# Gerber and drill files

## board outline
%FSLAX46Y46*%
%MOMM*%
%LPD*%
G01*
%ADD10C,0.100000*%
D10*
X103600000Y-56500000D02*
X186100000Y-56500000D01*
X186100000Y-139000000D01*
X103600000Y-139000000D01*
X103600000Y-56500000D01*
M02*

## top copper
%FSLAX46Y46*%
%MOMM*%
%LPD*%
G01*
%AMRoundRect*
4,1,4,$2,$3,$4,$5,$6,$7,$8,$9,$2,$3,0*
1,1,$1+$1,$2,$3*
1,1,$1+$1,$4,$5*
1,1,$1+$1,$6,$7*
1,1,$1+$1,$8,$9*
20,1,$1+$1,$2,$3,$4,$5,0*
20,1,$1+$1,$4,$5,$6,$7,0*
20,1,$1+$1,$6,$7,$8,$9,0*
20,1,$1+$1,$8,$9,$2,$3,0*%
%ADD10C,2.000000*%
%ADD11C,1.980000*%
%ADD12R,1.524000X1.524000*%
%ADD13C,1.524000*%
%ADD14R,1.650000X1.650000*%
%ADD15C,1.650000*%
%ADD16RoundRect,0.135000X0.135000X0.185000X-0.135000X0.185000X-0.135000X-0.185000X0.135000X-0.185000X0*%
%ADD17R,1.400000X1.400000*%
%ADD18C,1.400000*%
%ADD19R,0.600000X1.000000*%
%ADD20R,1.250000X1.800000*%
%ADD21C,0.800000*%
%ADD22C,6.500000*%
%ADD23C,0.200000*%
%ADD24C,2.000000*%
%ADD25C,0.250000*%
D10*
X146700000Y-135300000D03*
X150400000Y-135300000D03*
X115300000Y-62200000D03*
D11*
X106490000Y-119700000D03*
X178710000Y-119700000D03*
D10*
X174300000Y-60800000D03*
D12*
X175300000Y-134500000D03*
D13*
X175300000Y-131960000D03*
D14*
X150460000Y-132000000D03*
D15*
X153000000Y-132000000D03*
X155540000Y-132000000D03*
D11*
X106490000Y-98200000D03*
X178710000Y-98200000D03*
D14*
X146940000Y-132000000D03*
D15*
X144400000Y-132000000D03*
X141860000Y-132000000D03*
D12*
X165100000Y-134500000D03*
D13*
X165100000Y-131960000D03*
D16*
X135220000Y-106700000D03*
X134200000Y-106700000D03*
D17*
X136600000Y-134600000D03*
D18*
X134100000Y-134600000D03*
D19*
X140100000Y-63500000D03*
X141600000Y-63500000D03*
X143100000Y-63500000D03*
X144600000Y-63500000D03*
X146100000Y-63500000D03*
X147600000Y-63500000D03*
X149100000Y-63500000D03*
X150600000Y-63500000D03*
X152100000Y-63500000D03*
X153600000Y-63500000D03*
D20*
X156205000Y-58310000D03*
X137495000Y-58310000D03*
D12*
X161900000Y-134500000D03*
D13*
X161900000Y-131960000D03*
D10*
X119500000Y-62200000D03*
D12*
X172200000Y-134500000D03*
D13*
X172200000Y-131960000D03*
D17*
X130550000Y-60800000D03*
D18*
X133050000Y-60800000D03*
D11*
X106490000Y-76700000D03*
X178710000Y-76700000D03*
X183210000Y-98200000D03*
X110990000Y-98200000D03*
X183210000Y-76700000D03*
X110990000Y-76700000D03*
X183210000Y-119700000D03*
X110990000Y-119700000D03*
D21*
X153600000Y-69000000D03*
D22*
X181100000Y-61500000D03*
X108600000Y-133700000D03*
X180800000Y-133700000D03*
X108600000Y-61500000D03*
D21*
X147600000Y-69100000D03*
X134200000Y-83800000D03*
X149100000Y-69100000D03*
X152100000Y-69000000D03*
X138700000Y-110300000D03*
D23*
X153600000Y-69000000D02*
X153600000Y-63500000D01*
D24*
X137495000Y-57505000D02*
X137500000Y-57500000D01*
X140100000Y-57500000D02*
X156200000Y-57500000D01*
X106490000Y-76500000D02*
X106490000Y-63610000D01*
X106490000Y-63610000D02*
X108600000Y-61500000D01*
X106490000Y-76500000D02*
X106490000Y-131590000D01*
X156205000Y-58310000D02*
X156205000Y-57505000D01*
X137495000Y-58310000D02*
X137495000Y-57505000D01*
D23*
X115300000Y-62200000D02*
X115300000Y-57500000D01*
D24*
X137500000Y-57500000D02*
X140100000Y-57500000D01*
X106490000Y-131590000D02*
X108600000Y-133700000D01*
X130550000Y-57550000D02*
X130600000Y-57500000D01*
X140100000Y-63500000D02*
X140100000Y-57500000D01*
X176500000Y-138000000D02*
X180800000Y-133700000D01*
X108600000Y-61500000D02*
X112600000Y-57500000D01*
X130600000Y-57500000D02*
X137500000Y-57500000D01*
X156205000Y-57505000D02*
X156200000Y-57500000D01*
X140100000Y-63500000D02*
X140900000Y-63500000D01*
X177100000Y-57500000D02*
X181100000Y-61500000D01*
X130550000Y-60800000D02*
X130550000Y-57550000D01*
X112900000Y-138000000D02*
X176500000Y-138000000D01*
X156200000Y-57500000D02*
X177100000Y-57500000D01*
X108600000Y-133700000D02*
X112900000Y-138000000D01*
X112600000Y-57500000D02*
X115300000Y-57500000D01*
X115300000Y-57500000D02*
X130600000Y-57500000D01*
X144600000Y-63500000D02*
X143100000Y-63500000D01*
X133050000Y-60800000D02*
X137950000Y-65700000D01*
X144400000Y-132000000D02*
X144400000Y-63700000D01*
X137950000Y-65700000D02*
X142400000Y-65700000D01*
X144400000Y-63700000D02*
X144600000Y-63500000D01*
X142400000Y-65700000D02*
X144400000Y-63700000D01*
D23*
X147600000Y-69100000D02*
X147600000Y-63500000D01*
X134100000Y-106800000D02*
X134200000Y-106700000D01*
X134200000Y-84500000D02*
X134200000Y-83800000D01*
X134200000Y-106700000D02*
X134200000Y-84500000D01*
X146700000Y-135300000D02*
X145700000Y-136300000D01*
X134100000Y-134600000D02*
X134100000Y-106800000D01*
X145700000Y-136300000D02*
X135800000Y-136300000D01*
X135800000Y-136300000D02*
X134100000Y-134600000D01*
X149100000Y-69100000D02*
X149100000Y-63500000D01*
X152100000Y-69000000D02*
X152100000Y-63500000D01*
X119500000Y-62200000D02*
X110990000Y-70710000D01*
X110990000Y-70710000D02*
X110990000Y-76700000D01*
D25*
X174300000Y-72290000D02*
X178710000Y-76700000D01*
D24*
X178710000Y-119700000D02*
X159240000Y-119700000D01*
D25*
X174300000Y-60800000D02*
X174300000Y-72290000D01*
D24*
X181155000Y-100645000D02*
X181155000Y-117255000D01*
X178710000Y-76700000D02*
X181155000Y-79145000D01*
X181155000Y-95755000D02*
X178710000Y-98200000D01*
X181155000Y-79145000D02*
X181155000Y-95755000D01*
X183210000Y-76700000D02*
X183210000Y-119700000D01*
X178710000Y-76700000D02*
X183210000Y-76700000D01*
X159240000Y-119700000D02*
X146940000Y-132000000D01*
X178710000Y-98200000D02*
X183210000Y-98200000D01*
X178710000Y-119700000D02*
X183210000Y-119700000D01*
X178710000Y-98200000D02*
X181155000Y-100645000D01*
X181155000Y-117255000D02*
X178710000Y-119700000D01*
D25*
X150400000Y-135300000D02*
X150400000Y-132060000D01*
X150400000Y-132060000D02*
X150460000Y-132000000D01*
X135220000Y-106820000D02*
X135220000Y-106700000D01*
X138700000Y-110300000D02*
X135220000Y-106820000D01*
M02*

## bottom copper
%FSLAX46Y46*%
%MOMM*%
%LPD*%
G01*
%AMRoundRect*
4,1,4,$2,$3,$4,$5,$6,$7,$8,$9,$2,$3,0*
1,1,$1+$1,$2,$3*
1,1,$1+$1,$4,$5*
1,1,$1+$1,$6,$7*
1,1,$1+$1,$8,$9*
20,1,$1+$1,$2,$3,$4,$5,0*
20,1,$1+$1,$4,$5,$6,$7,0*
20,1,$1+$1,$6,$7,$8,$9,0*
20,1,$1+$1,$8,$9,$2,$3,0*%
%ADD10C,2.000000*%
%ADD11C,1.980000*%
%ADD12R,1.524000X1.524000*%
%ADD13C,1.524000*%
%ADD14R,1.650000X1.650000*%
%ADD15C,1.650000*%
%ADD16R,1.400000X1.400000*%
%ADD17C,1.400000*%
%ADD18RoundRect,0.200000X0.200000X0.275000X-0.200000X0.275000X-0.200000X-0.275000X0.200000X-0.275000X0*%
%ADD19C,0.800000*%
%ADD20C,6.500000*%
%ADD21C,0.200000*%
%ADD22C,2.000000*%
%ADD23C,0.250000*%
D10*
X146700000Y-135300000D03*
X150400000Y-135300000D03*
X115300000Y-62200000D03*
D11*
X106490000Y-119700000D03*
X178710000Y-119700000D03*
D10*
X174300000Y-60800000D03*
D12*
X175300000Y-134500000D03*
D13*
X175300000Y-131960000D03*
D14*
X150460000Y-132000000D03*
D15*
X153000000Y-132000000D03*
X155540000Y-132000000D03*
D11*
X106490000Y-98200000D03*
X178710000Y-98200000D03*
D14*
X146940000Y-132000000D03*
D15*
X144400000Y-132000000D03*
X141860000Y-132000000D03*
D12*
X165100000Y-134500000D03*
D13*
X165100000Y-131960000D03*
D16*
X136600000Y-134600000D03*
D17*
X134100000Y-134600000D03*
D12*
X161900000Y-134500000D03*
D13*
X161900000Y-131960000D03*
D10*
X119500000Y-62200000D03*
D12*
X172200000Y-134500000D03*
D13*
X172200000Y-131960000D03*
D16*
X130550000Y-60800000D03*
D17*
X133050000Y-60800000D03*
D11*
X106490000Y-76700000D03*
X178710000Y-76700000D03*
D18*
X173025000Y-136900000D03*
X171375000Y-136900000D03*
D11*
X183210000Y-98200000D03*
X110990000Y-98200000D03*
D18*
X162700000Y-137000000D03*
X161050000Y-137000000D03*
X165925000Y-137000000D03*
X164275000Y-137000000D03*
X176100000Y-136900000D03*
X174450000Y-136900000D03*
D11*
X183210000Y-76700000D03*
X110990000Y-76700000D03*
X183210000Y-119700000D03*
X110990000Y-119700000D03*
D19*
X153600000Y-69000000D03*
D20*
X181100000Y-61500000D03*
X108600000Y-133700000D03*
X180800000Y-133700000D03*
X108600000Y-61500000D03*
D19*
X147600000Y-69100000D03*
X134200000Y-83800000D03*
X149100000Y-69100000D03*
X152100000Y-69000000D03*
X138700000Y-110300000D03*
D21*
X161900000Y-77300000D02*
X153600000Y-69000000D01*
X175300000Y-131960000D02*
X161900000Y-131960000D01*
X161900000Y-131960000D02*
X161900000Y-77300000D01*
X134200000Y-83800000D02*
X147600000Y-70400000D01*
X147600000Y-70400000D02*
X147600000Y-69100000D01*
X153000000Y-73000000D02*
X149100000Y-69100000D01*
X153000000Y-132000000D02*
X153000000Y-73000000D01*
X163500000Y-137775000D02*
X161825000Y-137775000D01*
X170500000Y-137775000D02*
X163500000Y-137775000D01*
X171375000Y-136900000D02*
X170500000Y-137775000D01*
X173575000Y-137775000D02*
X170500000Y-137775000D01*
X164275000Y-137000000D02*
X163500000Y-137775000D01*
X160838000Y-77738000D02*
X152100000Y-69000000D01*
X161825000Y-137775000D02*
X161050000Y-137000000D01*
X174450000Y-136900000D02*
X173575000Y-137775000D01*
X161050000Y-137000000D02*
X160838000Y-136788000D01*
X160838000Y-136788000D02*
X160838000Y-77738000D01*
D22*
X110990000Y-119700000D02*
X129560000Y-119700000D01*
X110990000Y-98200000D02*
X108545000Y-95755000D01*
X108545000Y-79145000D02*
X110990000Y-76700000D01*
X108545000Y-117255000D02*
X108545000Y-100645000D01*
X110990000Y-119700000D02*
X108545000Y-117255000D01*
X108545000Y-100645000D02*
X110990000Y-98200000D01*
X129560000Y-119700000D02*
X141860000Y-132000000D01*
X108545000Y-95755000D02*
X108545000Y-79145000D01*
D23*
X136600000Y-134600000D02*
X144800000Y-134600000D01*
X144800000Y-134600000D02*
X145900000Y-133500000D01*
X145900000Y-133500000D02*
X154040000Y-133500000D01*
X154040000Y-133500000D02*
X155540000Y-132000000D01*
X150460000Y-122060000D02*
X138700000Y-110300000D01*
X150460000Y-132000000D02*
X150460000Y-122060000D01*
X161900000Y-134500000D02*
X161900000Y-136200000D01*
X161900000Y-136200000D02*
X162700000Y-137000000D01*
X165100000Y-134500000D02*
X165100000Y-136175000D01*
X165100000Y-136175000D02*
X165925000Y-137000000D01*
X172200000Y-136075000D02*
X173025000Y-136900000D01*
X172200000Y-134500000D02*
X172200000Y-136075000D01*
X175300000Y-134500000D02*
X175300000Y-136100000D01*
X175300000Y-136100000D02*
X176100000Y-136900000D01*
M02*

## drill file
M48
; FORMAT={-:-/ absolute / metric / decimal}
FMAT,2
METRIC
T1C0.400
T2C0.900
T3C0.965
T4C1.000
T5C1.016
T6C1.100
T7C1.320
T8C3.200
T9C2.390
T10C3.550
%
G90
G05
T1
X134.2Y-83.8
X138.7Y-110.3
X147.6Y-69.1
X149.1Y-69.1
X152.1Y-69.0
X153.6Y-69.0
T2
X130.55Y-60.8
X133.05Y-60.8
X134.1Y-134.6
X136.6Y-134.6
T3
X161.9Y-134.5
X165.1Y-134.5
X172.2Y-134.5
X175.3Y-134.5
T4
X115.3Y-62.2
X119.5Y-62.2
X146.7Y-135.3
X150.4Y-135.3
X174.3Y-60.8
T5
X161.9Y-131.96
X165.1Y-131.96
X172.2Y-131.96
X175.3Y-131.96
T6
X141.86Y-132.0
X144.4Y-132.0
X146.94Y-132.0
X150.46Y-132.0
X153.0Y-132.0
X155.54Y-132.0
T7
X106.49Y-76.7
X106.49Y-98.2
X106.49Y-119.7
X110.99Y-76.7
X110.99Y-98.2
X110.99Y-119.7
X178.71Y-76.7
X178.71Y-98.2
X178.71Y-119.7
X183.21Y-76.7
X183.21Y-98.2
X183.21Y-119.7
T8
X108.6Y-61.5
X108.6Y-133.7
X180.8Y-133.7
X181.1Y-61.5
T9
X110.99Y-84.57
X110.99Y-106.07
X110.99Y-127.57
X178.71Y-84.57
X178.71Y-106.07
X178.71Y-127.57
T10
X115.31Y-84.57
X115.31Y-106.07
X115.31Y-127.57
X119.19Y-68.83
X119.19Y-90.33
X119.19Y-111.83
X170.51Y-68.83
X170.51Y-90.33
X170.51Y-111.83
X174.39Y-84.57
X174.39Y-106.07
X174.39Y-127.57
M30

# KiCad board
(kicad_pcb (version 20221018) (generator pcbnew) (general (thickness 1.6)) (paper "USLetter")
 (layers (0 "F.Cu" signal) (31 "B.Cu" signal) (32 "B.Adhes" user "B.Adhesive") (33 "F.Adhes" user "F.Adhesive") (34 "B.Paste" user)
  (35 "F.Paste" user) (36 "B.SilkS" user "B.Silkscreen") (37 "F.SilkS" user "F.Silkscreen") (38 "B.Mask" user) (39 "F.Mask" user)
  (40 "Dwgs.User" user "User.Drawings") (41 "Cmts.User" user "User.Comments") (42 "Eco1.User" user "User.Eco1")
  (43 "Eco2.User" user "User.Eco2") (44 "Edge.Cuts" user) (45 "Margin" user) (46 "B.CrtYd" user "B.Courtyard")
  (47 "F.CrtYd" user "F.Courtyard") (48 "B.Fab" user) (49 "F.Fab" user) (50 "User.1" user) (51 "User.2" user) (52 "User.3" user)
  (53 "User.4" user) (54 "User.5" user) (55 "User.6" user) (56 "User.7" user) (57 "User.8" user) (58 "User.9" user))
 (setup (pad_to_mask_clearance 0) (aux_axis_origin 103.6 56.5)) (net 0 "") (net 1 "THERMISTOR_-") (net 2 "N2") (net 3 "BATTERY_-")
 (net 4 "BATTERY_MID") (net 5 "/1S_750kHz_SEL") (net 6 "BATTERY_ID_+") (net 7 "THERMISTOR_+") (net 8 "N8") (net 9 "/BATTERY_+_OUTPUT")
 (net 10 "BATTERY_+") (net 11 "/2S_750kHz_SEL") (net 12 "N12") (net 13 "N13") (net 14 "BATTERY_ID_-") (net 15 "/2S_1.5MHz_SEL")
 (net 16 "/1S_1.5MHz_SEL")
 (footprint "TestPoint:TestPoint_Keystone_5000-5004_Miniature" (layer "F.Cu") (at 146.7 135.3)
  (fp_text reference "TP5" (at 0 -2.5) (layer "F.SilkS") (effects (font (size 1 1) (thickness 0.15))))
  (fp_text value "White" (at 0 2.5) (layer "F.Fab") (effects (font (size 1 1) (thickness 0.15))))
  (pad "1" thru_hole circle (at 0 0) (size 2 2) (drill 1) (layers "*.Cu" "*.Mask") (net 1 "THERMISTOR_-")))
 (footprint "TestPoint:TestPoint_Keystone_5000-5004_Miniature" (layer "F.Cu") (at 150.4 135.3)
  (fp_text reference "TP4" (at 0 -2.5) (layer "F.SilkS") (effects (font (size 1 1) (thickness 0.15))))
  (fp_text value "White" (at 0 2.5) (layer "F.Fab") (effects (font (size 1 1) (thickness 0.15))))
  (pad "1" thru_hole circle (at 0 0) (size 2 2) (drill 1) (layers "*.Cu" "*.Mask") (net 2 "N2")))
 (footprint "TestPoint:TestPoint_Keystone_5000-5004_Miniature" (layer "F.Cu") (at 115.3 62.2)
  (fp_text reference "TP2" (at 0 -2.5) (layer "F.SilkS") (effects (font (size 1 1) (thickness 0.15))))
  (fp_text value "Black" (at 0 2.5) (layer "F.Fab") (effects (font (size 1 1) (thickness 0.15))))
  (pad "1" thru_hole circle (at 0 0) (size 2 2) (drill 1) (layers "*.Cu" "*.Mask") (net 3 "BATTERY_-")))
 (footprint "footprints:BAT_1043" (layer "F.Cu") (at 142.6 119.7)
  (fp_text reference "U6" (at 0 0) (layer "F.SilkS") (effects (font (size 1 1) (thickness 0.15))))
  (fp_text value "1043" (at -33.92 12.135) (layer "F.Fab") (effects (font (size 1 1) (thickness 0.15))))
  (pad "" np_thru_hole circle (at -27.29 7.87) (size 3.55 3.55) (drill 3.55) (layers "*.Cu" "*.Mask"))
  (pad "" np_thru_hole circle (at 27.91 -7.87) (size 3.55 3.55) (drill 3.55) (layers "*.Cu" "*.Mask"))
  (pad "" np_thru_hole circle (at 36.11 7.87) (size 2.39 2.39) (drill 2.39) (layers "*.Cu" "*.Mask"))
  (pad "N" thru_hole circle (at -36.11 0) (size 1.98 1.98) (drill 1.32) (layers "*.Cu" "*.Mask") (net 3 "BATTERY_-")
   (solder_mask_margin 0.102))
  (pad "P" thru_hole circle (at 36.11 0) (size 1.98 1.98) (drill 1.32) (layers "*.Cu" "*.Mask") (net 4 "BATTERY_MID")
   (solder_mask_margin 0.102)))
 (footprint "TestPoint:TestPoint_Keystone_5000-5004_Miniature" (layer "F.Cu") (at 174.3 60.8)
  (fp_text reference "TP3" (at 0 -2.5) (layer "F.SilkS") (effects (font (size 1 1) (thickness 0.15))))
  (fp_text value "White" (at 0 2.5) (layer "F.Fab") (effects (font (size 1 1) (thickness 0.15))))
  (pad "1" thru_hole circle (at 0 0) (size 2 2) (drill 1) (layers "*.Cu" "*.Mask") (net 4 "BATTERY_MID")))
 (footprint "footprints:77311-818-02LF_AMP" (layer "F.Cu") (at 175.3 134.5 -90)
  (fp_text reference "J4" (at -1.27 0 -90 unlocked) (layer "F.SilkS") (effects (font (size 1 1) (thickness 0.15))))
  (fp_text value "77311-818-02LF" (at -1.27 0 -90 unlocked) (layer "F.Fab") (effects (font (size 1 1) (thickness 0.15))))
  (pad "1" thru_hole rect (at 0 0 270) (size 1.524 1.524) (drill 0.9652) (layers "*.Cu" "*.Mask") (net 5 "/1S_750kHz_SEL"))
  (pad "2" thru_hole circle (at -2.54 0 270) (size 1.524 1.524) (drill 1.016) (layers "*.Cu" "*.Mask") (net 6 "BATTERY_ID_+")))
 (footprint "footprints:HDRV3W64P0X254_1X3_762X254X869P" (layer "F.Cu") (at 150.46 132)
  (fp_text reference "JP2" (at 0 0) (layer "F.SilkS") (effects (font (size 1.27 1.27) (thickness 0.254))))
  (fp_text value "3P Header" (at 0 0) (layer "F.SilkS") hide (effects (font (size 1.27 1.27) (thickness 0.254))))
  (pad "1" thru_hole rect (at 0 0) (size 1.65 1.65) (drill 1.1) (layers "*.Cu" "*.Mask") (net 2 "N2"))
  (pad "2" thru_hole circle (at 2.54 0) (size 1.65 1.65) (drill 1.1) (layers "*.Cu" "*.Mask") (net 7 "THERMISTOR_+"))
  (pad "3" thru_hole circle (at 5.08 0) (size 1.65 1.65) (drill 1.1) (layers "*.Cu" "*.Mask") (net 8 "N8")))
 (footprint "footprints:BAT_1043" (layer "F.Cu") (at 142.6 98.2)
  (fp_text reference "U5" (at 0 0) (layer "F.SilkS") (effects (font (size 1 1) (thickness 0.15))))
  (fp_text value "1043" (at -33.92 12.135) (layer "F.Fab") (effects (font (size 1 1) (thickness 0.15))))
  (pad "" np_thru_hole circle (at -27.29 7.87) (size 3.55 3.55) (drill 3.55) (layers "*.Cu" "*.Mask"))
  (pad "" np_thru_hole circle (at 27.91 -7.87) (size 3.55 3.55) (drill 3.55) (layers "*.Cu" "*.Mask"))
  (pad "" np_thru_hole circle (at 36.11 7.87) (size 2.39 2.39) (drill 2.39) (layers "*.Cu" "*.Mask"))
  (pad "N" thru_hole circle (at -36.11 0) (size 1.98 1.98) (drill 1.32) (layers "*.Cu" "*.Mask") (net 3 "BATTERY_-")
   (solder_mask_margin 0.102))
  (pad "P" thru_hole circle (at 36.11 0) (size 1.98 1.98) (drill 1.32) (layers "*.Cu" "*.Mask") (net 4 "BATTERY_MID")
   (solder_mask_margin 0.102)))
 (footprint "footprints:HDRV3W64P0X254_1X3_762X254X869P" (layer "F.Cu") (at 146.94 132 180)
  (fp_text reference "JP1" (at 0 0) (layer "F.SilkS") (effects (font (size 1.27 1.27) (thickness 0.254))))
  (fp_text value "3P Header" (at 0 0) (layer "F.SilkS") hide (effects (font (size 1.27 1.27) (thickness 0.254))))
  (pad "1" thru_hole rect (at 0 0 180) (size 1.65 1.65) (drill 1.1) (layers "*.Cu" "*.Mask") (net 4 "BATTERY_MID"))
  (pad "2" thru_hole circle (at 2.54 0 180) (size 1.65 1.65) (drill 1.1) (layers "*.Cu" "*.Mask") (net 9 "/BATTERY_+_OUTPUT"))
  (pad "3" thru_hole circle (at 5.08 0 180) (size 1.65 1.65) (drill 1.1) (layers "*.Cu" "*.Mask") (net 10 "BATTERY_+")))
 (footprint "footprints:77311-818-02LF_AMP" (layer "F.Cu") (at 165.1 134.5 -90)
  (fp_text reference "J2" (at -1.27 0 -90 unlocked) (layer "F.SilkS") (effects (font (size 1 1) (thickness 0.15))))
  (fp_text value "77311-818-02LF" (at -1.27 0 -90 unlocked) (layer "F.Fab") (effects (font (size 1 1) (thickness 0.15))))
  (pad "1" thru_hole rect (at 0 0 270) (size 1.524 1.524) (drill 0.9652) (layers "*.Cu" "*.Mask") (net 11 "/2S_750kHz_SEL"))
  (pad "2" thru_hole circle (at -2.54 0 270) (size 1.524 1.524) (drill 1.016) (layers "*.Cu" "*.Mask") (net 6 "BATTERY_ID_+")))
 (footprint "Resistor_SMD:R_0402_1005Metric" (layer "F.Cu") (at 134.71 106.7 180)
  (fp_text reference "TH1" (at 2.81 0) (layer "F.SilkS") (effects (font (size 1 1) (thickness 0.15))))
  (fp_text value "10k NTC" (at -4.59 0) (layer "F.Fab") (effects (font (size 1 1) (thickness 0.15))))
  (pad "1" smd roundrect (at -0.51 0 180) (size 0.54 0.64) (layers "F.Cu" "F.Paste" "F.Mask") (roundrect_rratio 0.25) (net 2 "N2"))
  (pad "2" smd roundrect (at 0.51 0 180) (size 0.54 0.64) (layers "F.Cu" "F.Paste" "F.Mask") (roundrect_rratio 0.25) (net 1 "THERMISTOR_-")))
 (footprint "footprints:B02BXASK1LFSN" (layer "F.Cu") (at 136.6 134.6)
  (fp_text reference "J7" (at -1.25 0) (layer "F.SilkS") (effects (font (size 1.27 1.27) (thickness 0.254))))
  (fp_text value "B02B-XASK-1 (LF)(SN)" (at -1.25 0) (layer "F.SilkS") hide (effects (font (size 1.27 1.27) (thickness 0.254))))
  (pad "1" thru_hole rect (at 0 0) (size 1.4 1.4) (drill 0.9) (layers "*.Cu" "*.Mask") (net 8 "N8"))
  (pad "2" thru_hole circle (at -2.5 0) (size 1.4 1.4) (drill 0.9) (layers "*.Cu" "*.Mask") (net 1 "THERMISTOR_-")))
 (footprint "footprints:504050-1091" (layer "F.Cu") (at 153.6 63.5)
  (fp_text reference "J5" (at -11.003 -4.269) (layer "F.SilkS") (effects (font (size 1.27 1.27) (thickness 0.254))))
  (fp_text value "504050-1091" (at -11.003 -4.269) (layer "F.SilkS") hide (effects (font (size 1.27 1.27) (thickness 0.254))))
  (pad "1" smd rect (at -13.5 0) (size 0.6 1) (layers "F.Cu" "F.Paste" "F.Mask") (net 3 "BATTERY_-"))
  (pad "2" smd rect (at -12 0) (size 0.6 1) (layers "F.Cu" "F.Paste" "F.Mask") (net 3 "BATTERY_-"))
  (pad "3" smd rect (at -10.5 0) (size 0.6 1) (layers "F.Cu" "F.Paste" "F.Mask") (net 9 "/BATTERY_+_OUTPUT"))
  (pad "4" smd rect (at -9 0) (size 0.6 1) (layers "F.Cu" "F.Paste" "F.Mask") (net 9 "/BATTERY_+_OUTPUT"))
  (pad "5" smd rect (at -7.5 0) (size 0.6 1) (layers "F.Cu" "F.Paste" "F.Mask") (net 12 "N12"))
  (pad "6" smd rect (at -6 0) (size 0.6 1) (layers "F.Cu" "F.Paste" "F.Mask") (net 1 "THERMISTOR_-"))
  (pad "7" smd rect (at -4.5 0) (size 0.6 1) (layers "F.Cu" "F.Paste" "F.Mask") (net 7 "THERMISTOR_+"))
  (pad "8" smd rect (at -3 0) (size 0.6 1) (layers "F.Cu" "F.Paste" "F.Mask") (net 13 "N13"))
  (pad "9" smd rect (at -1.5 0) (size 0.6 1) (layers "F.Cu" "F.Paste" "F.Mask") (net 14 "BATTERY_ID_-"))
  (pad "10" smd rect (at 0 0) (size 0.6 1) (layers "F.Cu" "F.Paste" "F.Mask") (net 6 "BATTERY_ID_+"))
  (pad "11" smd rect (at 2.605 -5.19) (size 1.25 1.8) (layers "F.Cu" "F.Paste" "F.Mask") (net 3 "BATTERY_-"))
  (pad "12" smd rect (at -16.105 -5.19) (size 1.25 1.8) (layers "F.Cu" "F.Paste" "F.Mask") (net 3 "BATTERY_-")))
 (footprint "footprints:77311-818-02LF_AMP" (layer "F.Cu") (at 161.9 134.5 -90)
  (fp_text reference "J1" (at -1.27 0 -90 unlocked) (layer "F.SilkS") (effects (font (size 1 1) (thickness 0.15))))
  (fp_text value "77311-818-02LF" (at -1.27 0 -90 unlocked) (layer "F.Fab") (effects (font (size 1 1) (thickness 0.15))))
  (pad "1" thru_hole rect (at 0 0 270) (size 1.524 1.524) (drill 0.9652) (layers "*.Cu" "*.Mask") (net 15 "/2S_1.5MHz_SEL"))
  (pad "2" thru_hole circle (at -2.54 0 270) (size 1.524 1.524) (drill 1.016) (layers "*.Cu" "*.Mask") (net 6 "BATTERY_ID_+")))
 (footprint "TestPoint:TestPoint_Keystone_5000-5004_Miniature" (layer "F.Cu") (at 119.5 62.2)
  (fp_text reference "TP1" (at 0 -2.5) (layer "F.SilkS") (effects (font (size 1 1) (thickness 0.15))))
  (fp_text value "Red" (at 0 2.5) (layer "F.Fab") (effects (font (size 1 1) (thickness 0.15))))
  (pad "1" thru_hole circle (at 0 0) (size 2 2) (drill 1) (layers "*.Cu" "*.Mask") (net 10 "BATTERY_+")))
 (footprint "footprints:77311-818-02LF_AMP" (layer "F.Cu") (at 172.2 134.5 -90)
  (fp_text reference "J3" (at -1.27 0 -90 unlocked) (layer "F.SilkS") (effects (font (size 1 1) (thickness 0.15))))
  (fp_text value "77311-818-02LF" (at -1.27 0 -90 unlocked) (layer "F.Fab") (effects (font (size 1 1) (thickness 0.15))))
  (pad "1" thru_hole rect (at 0 0 270) (size 1.524 1.524) (drill 0.9652) (layers "*.Cu" "*.Mask") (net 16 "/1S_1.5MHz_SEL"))
  (pad "2" thru_hole circle (at -2.54 0 270) (size 1.524 1.524) (drill 1.016) (layers "*.Cu" "*.Mask") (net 6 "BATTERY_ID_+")))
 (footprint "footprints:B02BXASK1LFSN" (layer "F.Cu") (at 130.55 60.8 180)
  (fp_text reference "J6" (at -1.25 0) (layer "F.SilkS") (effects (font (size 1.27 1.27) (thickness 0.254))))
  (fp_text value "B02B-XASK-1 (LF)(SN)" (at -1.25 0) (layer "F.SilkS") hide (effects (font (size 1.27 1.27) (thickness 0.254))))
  (pad "1" thru_hole rect (at 0 0 180) (size 1.4 1.4) (drill 0.9) (layers "*.Cu" "*.Mask") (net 3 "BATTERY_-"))
  (pad "2" thru_hole circle (at -2.5 0 180) (size 1.4 1.4) (drill 0.9) (layers "*.Cu" "*.Mask") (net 9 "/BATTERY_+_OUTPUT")))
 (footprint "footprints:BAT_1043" (layer "F.Cu") (at 142.6 76.7)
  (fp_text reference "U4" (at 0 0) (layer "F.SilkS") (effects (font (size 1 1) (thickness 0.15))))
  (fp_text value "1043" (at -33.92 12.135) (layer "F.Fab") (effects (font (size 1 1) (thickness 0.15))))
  (pad "" np_thru_hole circle (at -27.29 7.87) (size 3.55 3.55) (drill 3.55) (layers "*.Cu" "*.Mask"))
  (pad "" np_thru_hole circle (at 27.91 -7.87) (size 3.55 3.55) (drill 3.55) (layers "*.Cu" "*.Mask"))
  (pad "" np_thru_hole circle (at 36.11 7.87) (size 2.39 2.39) (drill 2.39) (layers "*.Cu" "*.Mask"))
  (pad "N" thru_hole circle (at -36.11 0) (size 1.98 1.98) (drill 1.32) (layers "*.Cu" "*.Mask") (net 3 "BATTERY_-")
   (solder_mask_margin 0.102))
  (pad "P" thru_hole circle (at 36.11 0) (size 1.98 1.98) (drill 1.32) (layers "*.Cu" "*.Mask") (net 4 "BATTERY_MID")
   (solder_mask_margin 0.102)))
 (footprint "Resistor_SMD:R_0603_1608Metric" (layer "B.Cu") (at 172.2 136.9 180)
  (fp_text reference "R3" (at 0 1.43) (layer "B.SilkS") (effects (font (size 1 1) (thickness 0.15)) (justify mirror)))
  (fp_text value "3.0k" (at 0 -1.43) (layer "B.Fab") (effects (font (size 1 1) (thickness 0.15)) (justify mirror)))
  (pad "1" smd roundrect (at -0.825 0 180) (size 0.8 0.95) (layers "B.Cu" "B.Paste" "B.Mask") (roundrect_rratio 0.25)
   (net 16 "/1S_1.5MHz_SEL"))
  (pad "2" smd roundrect (at 0.825 0 180) (size 0.8 0.95) (layers "B.Cu" "B.Paste" "B.Mask") (roundrect_rratio 0.25) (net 14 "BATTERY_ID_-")))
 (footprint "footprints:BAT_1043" (layer "B.Cu") (at 147.1 98.2 180)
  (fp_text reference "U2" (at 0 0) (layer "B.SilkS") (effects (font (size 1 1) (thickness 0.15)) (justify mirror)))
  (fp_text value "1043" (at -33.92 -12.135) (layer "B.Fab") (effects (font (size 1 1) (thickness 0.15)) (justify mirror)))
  (pad "" np_thru_hole circle (at -27.29 -7.87 180) (size 3.55 3.55) (drill 3.55) (layers "*.Cu" "*.Mask"))
  (pad "" np_thru_hole circle (at 27.91 7.87 180) (size 3.55 3.55) (drill 3.55) (layers "*.Cu" "*.Mask"))
  (pad "" np_thru_hole circle (at 36.11 -7.87 180) (size 2.39 2.39) (drill 2.39) (layers "*.Cu" "*.Mask"))
  (pad "N" thru_hole circle (at -36.11 0 180) (size 1.98 1.98) (drill 1.32) (layers "*.Cu" "*.Mask") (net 4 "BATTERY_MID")
   (solder_mask_margin 0.102))
  (pad "P" thru_hole circle (at 36.11 0 180) (size 1.98 1.98) (drill 1.32) (layers "*.Cu" "*.Mask") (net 10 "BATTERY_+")
   (solder_mask_margin 0.102)))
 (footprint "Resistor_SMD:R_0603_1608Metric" (layer "B.Cu") (at 161.875 137 180)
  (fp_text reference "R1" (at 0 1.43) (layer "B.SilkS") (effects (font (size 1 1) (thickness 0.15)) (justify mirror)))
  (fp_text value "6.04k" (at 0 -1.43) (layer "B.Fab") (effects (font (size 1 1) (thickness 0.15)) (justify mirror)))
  (pad "1" smd roundrect (at -0.825 0 180) (size 0.8 0.95) (layers "B.Cu" "B.Paste" "B.Mask") (roundrect_rratio 0.25)
   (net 15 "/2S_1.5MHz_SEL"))
  (pad "2" smd roundrect (at 0.825 0 180) (size 0.8 0.95) (layers "B.Cu" "B.Paste" "B.Mask") (roundrect_rratio 0.25) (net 14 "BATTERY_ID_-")))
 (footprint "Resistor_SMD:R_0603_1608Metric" (layer "B.Cu") (at 165.1 137 180)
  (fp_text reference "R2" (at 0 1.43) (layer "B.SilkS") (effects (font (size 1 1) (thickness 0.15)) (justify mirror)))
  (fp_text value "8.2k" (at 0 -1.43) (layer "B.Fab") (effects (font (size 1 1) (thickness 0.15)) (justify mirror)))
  (pad "1" smd roundrect (at -0.825 0 180) (size 0.8 0.95) (layers "B.Cu" "B.Paste" "B.Mask") (roundrect_rratio 0.25)
   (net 11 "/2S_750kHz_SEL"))
  (pad "2" smd roundrect (at 0.825 0 180) (size 0.8 0.95) (layers "B.Cu" "B.Paste" "B.Mask") (roundrect_rratio 0.25) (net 14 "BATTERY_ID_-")))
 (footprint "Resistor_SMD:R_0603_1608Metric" (layer "B.Cu") (at 175.275 136.9 180)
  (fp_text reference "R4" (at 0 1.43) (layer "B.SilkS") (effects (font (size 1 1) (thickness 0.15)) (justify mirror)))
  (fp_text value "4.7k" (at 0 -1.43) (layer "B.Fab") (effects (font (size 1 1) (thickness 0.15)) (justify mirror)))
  (pad "1" smd roundrect (at -0.825 0 180) (size 0.8 0.95) (layers "B.Cu" "B.Paste" "B.Mask") (roundrect_rratio 0.25)
   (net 5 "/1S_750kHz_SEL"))
  (pad "2" smd roundrect (at 0.825 0 180) (size 0.8 0.95) (layers "B.Cu" "B.Paste" "B.Mask") (roundrect_rratio 0.25) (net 14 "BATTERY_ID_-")))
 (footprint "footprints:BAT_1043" (layer "B.Cu") (at 147.1 76.7 180)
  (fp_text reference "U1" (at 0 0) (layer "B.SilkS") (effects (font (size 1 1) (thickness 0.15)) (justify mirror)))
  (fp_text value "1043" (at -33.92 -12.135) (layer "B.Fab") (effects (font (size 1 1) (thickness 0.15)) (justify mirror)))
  (pad "" np_thru_hole circle (at -27.29 -7.87 180) (size 3.55 3.55) (drill 3.55) (layers "*.Cu" "*.Mask"))
  (pad "" np_thru_hole circle (at 27.91 7.87 180) (size 3.55 3.55) (drill 3.55) (layers "*.Cu" "*.Mask"))
  (pad "" np_thru_hole circle (at 36.11 -7.87 180) (size 2.39 2.39) (drill 2.39) (layers "*.Cu" "*.Mask"))
  (pad "N" thru_hole circle (at -36.11 0 180) (size 1.98 1.98) (drill 1.32) (layers "*.Cu" "*.Mask") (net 4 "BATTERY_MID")
   (solder_mask_margin 0.102))
  (pad "P" thru_hole circle (at 36.11 0 180) (size 1.98 1.98) (drill 1.32) (layers "*.Cu" "*.Mask") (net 10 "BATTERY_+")
   (solder_mask_margin 0.102)))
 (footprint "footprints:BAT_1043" (layer "B.Cu") (at 147.1 119.7 180)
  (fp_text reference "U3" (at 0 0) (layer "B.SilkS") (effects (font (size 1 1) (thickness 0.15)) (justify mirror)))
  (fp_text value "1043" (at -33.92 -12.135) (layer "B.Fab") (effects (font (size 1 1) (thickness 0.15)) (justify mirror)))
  (pad "" np_thru_hole circle (at -27.29 -7.87 180) (size 3.55 3.55) (drill 3.55) (layers "*.Cu" "*.Mask"))
  (pad "" np_thru_hole circle (at 27.91 7.87 180) (size 3.55 3.55) (drill 3.55) (layers "*.Cu" "*.Mask"))
  (pad "" np_thru_hole circle (at 36.11 -7.87 180) (size 2.39 2.39) (drill 2.39) (layers "*.Cu" "*.Mask"))
  (pad "N" thru_hole circle (at -36.11 0 180) (size 1.98 1.98) (drill 1.32) (layers "*.Cu" "*.Mask") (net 4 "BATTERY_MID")
   (solder_mask_margin 0.102))
  (pad "P" thru_hole circle (at 36.11 0 180) (size 1.98 1.98) (drill 1.32) (layers "*.Cu" "*.Mask") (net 10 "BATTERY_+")
   (solder_mask_margin 0.102)))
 (gr_rect (start 103.6 56.5) (end 186.1 139) (stroke (width 0.1) (type default)) (fill none) (layer "Edge.Cuts"))
 (segment (start 153.6 69) (end 153.6 63.5) (width 0.2) (layer "F.Cu") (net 6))
 (via (at 153.6 69) (size 0.8) (drill 0.4) (layers "F.Cu" "B.Cu") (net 6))
 (segment (start 161.9 77.3) (end 153.6 69) (width 0.2) (layer "B.Cu") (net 6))
 (segment (start 175.3 131.96) (end 161.9 131.96) (width 0.2) (layer "B.Cu") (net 6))
 (segment (start 161.9 131.96) (end 161.9 77.3) (width 0.2) (layer "B.Cu") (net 6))
 (segment (start 137.495 57.505) (end 137.5 57.5) (width 2) (layer "F.Cu") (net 3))
 (segment (start 140.1 57.5) (end 156.2 57.5) (width 2) (layer "F.Cu") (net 3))
 (segment (start 106.49 76.5) (end 106.49 63.61) (width 2) (layer "F.Cu") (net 3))
 (segment (start 106.49 63.61) (end 108.6 61.5) (width 2) (layer "F.Cu") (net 3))
 (segment (start 106.49 76.5) (end 106.49 131.59) (width 2) (layer "F.Cu") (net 3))
 (segment (start 156.205 58.31) (end 156.205 57.505) (width 2) (layer "F.Cu") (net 3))
 (segment (start 137.495 58.31) (end 137.495 57.505) (width 2) (layer "F.Cu") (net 3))
 (segment (start 115.3 62.2) (end 115.3 57.5) (width 0.2) (layer "F.Cu") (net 3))
 (segment (start 137.5 57.5) (end 140.1 57.5) (width 2) (layer "F.Cu") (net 3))
 (segment (start 106.49 131.59) (end 108.6 133.7) (width 2) (layer "F.Cu") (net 3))
 (segment (start 130.55 57.55) (end 130.6 57.5) (width 2) (layer "F.Cu") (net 3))
 (segment (start 140.1 63.5) (end 140.1 57.5) (width 2) (layer "F.Cu") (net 3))
 (segment (start 176.5 138) (end 180.8 133.7) (width 2) (layer "F.Cu") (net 3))
 (segment (start 108.6 61.5) (end 112.6 57.5) (width 2) (layer "F.Cu") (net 3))
 (segment (start 130.6 57.5) (end 137.5 57.5) (width 2) (layer "F.Cu") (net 3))
 (segment (start 156.205 57.505) (end 156.2 57.5) (width 2) (layer "F.Cu") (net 3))
 (segment (start 140.1 63.5) (end 140.9 63.5) (width 2) (layer "F.Cu") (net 3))
 (segment (start 177.1 57.5) (end 181.1 61.5) (width 2) (layer "F.Cu") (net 3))
 (segment (start 130.55 60.8) (end 130.55 57.55) (width 2) (layer "F.Cu") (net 3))
 (segment (start 112.9 138) (end 176.5 138) (width 2) (layer "F.Cu") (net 3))
 (segment (start 156.2 57.5) (end 177.1 57.5) (width 2) (layer "F.Cu") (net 3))
 (segment (start 108.6 133.7) (end 112.9 138) (width 2) (layer "F.Cu") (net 3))
 (segment (start 112.6 57.5) (end 115.3 57.5) (width 2) (layer "F.Cu") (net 3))
 (segment (start 115.3 57.5) (end 130.6 57.5) (width 2) (layer "F.Cu") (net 3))
 (via (at 181.1 61.5) (size 6.5) (drill 3.2) (layers "F.Cu" "B.Cu") (free) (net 3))
 (via (at 108.6 133.7) (size 6.5) (drill 3.2) (layers "F.Cu" "B.Cu") (free) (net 3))
 (via (at 180.8 133.7) (size 6.5) (drill 3.2) (layers "F.Cu" "B.Cu") (free) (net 3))
 (via (at 108.6 61.5) (size 6.5) (drill 3.2) (layers "F.Cu" "B.Cu") (free) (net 3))
 (segment (start 144.6 63.5) (end 143.1 63.5) (width 2) (layer "F.Cu") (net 9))
 (segment (start 133.05 60.8) (end 137.95 65.7) (width 2) (layer "F.Cu") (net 9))
 (segment (start 144.4 132) (end 144.4 63.7) (width 2) (layer "F.Cu") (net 9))
 (segment (start 137.95 65.7) (end 142.4 65.7) (width 2) (layer "F.Cu") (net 9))
 (segment (start 144.4 63.7) (end 144.6 63.5) (width 2) (layer "F.Cu") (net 9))
 (segment (start 142.4 65.7) (end 144.4 63.7) (width 2) (layer "F.Cu") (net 9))
 (segment (start 147.6 69.1) (end 147.6 63.5) (width 0.2) (layer "F.Cu") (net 1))
 (segment (start 134.1 106.8) (end 134.2 106.7) (width 0.2) (layer "F.Cu") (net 1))
 (segment (start 134.2 84.5) (end 134.2 83.8) (width 0.2) (layer "F.Cu") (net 1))
 (segment (start 134.2 106.7) (end 134.2 84.5) (width 0.2) (layer "F.Cu") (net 1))
 (segment (start 146.7 135.3) (end 145.7 136.3) (width 0.2) (layer "F.Cu") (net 1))
 (segment (start 134.1 134.6) (end 134.1 106.8) (width 0.2) (layer "F.Cu") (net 1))
 (segment (start 145.7 136.3) (end 135.8 136.3) (width 0.2) (layer "F.Cu") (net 1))
 (segment (start 135.8 136.3) (end 134.1 134.6) (width 0.2) (layer "F.Cu") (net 1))
 (via (at 147.6 69.1) (size 0.8) (drill 0.4) (layers "F.Cu" "B.Cu") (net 1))
 (via (at 134.2 83.8) (size 0.8) (drill 0.4) (layers "F.Cu" "B.Cu") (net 1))
 (segment (start 134.2 83.8) (end 147.6 70.4) (width 0.2) (layer "B.Cu") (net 1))
 (segment (start 147.6 70.4) (end 147.6 69.1) (width 0.2) (layer "B.Cu") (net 1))
 (segment (start 149.1 69.1) (end 149.1 63.5) (width 0.2) (layer "F.Cu") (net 7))
 (via (at 149.1 69.1) (size 0.8) (drill 0.4) (layers "F.Cu" "B.Cu") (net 7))
 (segment (start 153 73) (end 149.1 69.1) (width 0.2) (layer "B.Cu") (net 7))
 (segment (start 153 132) (end 153 73) (width 0.2) (layer "B.Cu") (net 7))
 (segment (start 152.1 69) (end 152.1 63.5) (width 0.2) (layer "F.Cu") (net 14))
 (via (at 152.1 69) (size 0.8) (drill 0.4) (layers "F.Cu" "B.Cu") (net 14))
 (segment (start 163.5 137.775) (end 161.825 137.775) (width 0.2) (layer "B.Cu") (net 14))
 (segment (start 170.5 137.775) (end 163.5 137.775) (width 0.2) (layer "B.Cu") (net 14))
 (segment (start 171.375 136.9) (end 170.5 137.775) (width 0.2) (layer "B.Cu") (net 14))
 (segment (start 173.575 137.775) (end 170.5 137.775) (width 0.2) (layer "B.Cu") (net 14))
 (segment (start 164.275 137) (end 163.5 137.775) (width 0.2) (layer "B.Cu") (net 14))
 (segment (start 160.838 77.738) (end 152.1 69) (width 0.2) (layer "B.Cu") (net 14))
 (segment (start 161.825 137.775) (end 161.05 137) (width 0.2) (layer "B.Cu") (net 14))
 (segment (start 174.45 136.9) (end 173.575 137.775) (width 0.2) (layer "B.Cu") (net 14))
 (segment (start 161.05 137) (end 160.838 136.788) (width 0.2) (layer "B.Cu") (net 14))
 (segment (start 160.838 136.788) (end 160.838 77.738) (width 0.2) (layer "B.Cu") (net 14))
 (segment (start 119.5 62.2) (end 110.99 70.71) (width 0.2) (layer "F.Cu") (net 10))
 (segment (start 110.99 70.71) (end 110.99 76.7) (width 0.2) (layer "F.Cu") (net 10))
 (segment (start 110.99 119.7) (end 129.56 119.7) (width 2) (layer "B.Cu") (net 10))
 (segment (start 110.99 98.2) (end 108.545 95.755) (width 2) (layer "B.Cu") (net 10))
 (segment (start 108.545 79.145) (end 110.99 76.7) (width 2) (layer "B.Cu") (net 10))
 (segment (start 108.545 117.255) (end 108.545 100.645) (width 2) (layer "B.Cu") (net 10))
 (segment (start 110.99 119.7) (end 108.545 117.255) (width 2) (layer "B.Cu") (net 10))
 (segment (start 108.545 100.645) (end 110.99 98.2) (width 2) (layer "B.Cu") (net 10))
 (segment (start 129.56 119.7) (end 141.86 132) (width 2) (layer "B.Cu") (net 10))
 (segment (start 108.545 95.755) (end 108.545 79.145) (width 2) (layer "B.Cu") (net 10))
 (segment (start 136.6 134.6) (end 144.8 134.6) (width 0.25) (layer "B.Cu") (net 8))
 (segment (start 144.8 134.6) (end 145.9 133.5) (width 0.25) (layer "B.Cu") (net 8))
 (segment (start 145.9 133.5) (end 154.04 133.5) (width 0.25) (layer "B.Cu") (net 8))
 (segment (start 154.04 133.5) (end 155.54 132) (width 0.25) (layer "B.Cu") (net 8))
 (segment (start 174.3 72.29) (end 178.71 76.7) (width 0.25) (layer "F.Cu") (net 4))
 (segment (start 178.71 119.7) (end 159.24 119.7) (width 2) (layer "F.Cu") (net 4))
 (segment (start 174.3 60.8) (end 174.3 72.29) (width 0.25) (layer "F.Cu") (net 4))
 (segment (start 181.155 100.645) (end 181.155 117.255) (width 2) (layer "F.Cu") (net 4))
 (segment (start 178.71 76.7) (end 181.155 79.145) (width 2) (layer "F.Cu") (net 4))
 (segment (start 181.155 95.755) (end 178.71 98.2) (width 2) (layer "F.Cu") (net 4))
 (segment (start 181.155 79.145) (end 181.155 95.755) (width 2) (layer "F.Cu") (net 4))
 (segment (start 183.21 76.7) (end 183.21 119.7) (width 2) (layer "F.Cu") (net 4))
 (segment (start 178.71 76.7) (end 183.21 76.7) (width 2) (layer "F.Cu") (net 4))
 (segment (start 159.24 119.7) (end 146.94 132) (width 2) (layer "F.Cu") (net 4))
 (segment (start 178.71 98.2) (end 183.21 98.2) (width 2) (layer "F.Cu") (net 4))
 (segment (start 178.71 119.7) (end 183.21 119.7) (width 2) (layer "F.Cu") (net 4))
 (segment (start 178.71 98.2) (end 181.155 100.645) (width 2) (layer "F.Cu") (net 4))
 (segment (start 181.155 117.255) (end 178.71 119.7) (width 2) (layer "F.Cu") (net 4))
 (segment (start 150.4 135.3) (end 150.4 132.06) (width 0.25) (layer "F.Cu") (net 2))
 (segment (start 150.4 132.06) (end 150.46 132) (width 0.25) (layer "F.Cu") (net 2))
 (segment (start 135.22 106.82) (end 135.22 106.7) (width 0.25) (layer "F.Cu") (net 2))
 (segment (start 138.7 110.3) (end 135.22 106.82) (width 0.25) (layer "F.Cu") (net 2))
 (via (at 138.7 110.3) (size 0.8) (drill 0.4) (layers "F.Cu" "B.Cu") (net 2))
 (segment (start 150.46 122.06) (end 138.7 110.3) (width 0.25) (layer "B.Cu") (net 2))
 (segment (start 150.46 132) (end 150.46 122.06) (width 0.25) (layer "B.Cu") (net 2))
 (segment (start 161.9 134.5) (end 161.9 136.2) (width 0.25) (layer "B.Cu") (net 15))
 (segment (start 161.9 136.2) (end 162.7 137) (width 0.25) (layer "B.Cu") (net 15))
 (segment (start 165.1 134.5) (end 165.1 136.175) (width 0.25) (layer "B.Cu") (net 11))
 (segment (start 165.1 136.175) (end 165.925 137) (width 0.25) (layer "B.Cu") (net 11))
 (segment (start 172.2 136.075) (end 173.025 136.9) (width 0.25) (layer "B.Cu") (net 16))
 (segment (start 172.2 134.5) (end 172.2 136.075) (width 0.25) (layer "B.Cu") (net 16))
 (segment (start 175.3 134.5) (end 175.3 136.1) (width 0.25) (layer "B.Cu") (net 5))
 (segment (start 175.3 136.1) (end 176.1 136.9) (width 0.25) (layer "B.Cu") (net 5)))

